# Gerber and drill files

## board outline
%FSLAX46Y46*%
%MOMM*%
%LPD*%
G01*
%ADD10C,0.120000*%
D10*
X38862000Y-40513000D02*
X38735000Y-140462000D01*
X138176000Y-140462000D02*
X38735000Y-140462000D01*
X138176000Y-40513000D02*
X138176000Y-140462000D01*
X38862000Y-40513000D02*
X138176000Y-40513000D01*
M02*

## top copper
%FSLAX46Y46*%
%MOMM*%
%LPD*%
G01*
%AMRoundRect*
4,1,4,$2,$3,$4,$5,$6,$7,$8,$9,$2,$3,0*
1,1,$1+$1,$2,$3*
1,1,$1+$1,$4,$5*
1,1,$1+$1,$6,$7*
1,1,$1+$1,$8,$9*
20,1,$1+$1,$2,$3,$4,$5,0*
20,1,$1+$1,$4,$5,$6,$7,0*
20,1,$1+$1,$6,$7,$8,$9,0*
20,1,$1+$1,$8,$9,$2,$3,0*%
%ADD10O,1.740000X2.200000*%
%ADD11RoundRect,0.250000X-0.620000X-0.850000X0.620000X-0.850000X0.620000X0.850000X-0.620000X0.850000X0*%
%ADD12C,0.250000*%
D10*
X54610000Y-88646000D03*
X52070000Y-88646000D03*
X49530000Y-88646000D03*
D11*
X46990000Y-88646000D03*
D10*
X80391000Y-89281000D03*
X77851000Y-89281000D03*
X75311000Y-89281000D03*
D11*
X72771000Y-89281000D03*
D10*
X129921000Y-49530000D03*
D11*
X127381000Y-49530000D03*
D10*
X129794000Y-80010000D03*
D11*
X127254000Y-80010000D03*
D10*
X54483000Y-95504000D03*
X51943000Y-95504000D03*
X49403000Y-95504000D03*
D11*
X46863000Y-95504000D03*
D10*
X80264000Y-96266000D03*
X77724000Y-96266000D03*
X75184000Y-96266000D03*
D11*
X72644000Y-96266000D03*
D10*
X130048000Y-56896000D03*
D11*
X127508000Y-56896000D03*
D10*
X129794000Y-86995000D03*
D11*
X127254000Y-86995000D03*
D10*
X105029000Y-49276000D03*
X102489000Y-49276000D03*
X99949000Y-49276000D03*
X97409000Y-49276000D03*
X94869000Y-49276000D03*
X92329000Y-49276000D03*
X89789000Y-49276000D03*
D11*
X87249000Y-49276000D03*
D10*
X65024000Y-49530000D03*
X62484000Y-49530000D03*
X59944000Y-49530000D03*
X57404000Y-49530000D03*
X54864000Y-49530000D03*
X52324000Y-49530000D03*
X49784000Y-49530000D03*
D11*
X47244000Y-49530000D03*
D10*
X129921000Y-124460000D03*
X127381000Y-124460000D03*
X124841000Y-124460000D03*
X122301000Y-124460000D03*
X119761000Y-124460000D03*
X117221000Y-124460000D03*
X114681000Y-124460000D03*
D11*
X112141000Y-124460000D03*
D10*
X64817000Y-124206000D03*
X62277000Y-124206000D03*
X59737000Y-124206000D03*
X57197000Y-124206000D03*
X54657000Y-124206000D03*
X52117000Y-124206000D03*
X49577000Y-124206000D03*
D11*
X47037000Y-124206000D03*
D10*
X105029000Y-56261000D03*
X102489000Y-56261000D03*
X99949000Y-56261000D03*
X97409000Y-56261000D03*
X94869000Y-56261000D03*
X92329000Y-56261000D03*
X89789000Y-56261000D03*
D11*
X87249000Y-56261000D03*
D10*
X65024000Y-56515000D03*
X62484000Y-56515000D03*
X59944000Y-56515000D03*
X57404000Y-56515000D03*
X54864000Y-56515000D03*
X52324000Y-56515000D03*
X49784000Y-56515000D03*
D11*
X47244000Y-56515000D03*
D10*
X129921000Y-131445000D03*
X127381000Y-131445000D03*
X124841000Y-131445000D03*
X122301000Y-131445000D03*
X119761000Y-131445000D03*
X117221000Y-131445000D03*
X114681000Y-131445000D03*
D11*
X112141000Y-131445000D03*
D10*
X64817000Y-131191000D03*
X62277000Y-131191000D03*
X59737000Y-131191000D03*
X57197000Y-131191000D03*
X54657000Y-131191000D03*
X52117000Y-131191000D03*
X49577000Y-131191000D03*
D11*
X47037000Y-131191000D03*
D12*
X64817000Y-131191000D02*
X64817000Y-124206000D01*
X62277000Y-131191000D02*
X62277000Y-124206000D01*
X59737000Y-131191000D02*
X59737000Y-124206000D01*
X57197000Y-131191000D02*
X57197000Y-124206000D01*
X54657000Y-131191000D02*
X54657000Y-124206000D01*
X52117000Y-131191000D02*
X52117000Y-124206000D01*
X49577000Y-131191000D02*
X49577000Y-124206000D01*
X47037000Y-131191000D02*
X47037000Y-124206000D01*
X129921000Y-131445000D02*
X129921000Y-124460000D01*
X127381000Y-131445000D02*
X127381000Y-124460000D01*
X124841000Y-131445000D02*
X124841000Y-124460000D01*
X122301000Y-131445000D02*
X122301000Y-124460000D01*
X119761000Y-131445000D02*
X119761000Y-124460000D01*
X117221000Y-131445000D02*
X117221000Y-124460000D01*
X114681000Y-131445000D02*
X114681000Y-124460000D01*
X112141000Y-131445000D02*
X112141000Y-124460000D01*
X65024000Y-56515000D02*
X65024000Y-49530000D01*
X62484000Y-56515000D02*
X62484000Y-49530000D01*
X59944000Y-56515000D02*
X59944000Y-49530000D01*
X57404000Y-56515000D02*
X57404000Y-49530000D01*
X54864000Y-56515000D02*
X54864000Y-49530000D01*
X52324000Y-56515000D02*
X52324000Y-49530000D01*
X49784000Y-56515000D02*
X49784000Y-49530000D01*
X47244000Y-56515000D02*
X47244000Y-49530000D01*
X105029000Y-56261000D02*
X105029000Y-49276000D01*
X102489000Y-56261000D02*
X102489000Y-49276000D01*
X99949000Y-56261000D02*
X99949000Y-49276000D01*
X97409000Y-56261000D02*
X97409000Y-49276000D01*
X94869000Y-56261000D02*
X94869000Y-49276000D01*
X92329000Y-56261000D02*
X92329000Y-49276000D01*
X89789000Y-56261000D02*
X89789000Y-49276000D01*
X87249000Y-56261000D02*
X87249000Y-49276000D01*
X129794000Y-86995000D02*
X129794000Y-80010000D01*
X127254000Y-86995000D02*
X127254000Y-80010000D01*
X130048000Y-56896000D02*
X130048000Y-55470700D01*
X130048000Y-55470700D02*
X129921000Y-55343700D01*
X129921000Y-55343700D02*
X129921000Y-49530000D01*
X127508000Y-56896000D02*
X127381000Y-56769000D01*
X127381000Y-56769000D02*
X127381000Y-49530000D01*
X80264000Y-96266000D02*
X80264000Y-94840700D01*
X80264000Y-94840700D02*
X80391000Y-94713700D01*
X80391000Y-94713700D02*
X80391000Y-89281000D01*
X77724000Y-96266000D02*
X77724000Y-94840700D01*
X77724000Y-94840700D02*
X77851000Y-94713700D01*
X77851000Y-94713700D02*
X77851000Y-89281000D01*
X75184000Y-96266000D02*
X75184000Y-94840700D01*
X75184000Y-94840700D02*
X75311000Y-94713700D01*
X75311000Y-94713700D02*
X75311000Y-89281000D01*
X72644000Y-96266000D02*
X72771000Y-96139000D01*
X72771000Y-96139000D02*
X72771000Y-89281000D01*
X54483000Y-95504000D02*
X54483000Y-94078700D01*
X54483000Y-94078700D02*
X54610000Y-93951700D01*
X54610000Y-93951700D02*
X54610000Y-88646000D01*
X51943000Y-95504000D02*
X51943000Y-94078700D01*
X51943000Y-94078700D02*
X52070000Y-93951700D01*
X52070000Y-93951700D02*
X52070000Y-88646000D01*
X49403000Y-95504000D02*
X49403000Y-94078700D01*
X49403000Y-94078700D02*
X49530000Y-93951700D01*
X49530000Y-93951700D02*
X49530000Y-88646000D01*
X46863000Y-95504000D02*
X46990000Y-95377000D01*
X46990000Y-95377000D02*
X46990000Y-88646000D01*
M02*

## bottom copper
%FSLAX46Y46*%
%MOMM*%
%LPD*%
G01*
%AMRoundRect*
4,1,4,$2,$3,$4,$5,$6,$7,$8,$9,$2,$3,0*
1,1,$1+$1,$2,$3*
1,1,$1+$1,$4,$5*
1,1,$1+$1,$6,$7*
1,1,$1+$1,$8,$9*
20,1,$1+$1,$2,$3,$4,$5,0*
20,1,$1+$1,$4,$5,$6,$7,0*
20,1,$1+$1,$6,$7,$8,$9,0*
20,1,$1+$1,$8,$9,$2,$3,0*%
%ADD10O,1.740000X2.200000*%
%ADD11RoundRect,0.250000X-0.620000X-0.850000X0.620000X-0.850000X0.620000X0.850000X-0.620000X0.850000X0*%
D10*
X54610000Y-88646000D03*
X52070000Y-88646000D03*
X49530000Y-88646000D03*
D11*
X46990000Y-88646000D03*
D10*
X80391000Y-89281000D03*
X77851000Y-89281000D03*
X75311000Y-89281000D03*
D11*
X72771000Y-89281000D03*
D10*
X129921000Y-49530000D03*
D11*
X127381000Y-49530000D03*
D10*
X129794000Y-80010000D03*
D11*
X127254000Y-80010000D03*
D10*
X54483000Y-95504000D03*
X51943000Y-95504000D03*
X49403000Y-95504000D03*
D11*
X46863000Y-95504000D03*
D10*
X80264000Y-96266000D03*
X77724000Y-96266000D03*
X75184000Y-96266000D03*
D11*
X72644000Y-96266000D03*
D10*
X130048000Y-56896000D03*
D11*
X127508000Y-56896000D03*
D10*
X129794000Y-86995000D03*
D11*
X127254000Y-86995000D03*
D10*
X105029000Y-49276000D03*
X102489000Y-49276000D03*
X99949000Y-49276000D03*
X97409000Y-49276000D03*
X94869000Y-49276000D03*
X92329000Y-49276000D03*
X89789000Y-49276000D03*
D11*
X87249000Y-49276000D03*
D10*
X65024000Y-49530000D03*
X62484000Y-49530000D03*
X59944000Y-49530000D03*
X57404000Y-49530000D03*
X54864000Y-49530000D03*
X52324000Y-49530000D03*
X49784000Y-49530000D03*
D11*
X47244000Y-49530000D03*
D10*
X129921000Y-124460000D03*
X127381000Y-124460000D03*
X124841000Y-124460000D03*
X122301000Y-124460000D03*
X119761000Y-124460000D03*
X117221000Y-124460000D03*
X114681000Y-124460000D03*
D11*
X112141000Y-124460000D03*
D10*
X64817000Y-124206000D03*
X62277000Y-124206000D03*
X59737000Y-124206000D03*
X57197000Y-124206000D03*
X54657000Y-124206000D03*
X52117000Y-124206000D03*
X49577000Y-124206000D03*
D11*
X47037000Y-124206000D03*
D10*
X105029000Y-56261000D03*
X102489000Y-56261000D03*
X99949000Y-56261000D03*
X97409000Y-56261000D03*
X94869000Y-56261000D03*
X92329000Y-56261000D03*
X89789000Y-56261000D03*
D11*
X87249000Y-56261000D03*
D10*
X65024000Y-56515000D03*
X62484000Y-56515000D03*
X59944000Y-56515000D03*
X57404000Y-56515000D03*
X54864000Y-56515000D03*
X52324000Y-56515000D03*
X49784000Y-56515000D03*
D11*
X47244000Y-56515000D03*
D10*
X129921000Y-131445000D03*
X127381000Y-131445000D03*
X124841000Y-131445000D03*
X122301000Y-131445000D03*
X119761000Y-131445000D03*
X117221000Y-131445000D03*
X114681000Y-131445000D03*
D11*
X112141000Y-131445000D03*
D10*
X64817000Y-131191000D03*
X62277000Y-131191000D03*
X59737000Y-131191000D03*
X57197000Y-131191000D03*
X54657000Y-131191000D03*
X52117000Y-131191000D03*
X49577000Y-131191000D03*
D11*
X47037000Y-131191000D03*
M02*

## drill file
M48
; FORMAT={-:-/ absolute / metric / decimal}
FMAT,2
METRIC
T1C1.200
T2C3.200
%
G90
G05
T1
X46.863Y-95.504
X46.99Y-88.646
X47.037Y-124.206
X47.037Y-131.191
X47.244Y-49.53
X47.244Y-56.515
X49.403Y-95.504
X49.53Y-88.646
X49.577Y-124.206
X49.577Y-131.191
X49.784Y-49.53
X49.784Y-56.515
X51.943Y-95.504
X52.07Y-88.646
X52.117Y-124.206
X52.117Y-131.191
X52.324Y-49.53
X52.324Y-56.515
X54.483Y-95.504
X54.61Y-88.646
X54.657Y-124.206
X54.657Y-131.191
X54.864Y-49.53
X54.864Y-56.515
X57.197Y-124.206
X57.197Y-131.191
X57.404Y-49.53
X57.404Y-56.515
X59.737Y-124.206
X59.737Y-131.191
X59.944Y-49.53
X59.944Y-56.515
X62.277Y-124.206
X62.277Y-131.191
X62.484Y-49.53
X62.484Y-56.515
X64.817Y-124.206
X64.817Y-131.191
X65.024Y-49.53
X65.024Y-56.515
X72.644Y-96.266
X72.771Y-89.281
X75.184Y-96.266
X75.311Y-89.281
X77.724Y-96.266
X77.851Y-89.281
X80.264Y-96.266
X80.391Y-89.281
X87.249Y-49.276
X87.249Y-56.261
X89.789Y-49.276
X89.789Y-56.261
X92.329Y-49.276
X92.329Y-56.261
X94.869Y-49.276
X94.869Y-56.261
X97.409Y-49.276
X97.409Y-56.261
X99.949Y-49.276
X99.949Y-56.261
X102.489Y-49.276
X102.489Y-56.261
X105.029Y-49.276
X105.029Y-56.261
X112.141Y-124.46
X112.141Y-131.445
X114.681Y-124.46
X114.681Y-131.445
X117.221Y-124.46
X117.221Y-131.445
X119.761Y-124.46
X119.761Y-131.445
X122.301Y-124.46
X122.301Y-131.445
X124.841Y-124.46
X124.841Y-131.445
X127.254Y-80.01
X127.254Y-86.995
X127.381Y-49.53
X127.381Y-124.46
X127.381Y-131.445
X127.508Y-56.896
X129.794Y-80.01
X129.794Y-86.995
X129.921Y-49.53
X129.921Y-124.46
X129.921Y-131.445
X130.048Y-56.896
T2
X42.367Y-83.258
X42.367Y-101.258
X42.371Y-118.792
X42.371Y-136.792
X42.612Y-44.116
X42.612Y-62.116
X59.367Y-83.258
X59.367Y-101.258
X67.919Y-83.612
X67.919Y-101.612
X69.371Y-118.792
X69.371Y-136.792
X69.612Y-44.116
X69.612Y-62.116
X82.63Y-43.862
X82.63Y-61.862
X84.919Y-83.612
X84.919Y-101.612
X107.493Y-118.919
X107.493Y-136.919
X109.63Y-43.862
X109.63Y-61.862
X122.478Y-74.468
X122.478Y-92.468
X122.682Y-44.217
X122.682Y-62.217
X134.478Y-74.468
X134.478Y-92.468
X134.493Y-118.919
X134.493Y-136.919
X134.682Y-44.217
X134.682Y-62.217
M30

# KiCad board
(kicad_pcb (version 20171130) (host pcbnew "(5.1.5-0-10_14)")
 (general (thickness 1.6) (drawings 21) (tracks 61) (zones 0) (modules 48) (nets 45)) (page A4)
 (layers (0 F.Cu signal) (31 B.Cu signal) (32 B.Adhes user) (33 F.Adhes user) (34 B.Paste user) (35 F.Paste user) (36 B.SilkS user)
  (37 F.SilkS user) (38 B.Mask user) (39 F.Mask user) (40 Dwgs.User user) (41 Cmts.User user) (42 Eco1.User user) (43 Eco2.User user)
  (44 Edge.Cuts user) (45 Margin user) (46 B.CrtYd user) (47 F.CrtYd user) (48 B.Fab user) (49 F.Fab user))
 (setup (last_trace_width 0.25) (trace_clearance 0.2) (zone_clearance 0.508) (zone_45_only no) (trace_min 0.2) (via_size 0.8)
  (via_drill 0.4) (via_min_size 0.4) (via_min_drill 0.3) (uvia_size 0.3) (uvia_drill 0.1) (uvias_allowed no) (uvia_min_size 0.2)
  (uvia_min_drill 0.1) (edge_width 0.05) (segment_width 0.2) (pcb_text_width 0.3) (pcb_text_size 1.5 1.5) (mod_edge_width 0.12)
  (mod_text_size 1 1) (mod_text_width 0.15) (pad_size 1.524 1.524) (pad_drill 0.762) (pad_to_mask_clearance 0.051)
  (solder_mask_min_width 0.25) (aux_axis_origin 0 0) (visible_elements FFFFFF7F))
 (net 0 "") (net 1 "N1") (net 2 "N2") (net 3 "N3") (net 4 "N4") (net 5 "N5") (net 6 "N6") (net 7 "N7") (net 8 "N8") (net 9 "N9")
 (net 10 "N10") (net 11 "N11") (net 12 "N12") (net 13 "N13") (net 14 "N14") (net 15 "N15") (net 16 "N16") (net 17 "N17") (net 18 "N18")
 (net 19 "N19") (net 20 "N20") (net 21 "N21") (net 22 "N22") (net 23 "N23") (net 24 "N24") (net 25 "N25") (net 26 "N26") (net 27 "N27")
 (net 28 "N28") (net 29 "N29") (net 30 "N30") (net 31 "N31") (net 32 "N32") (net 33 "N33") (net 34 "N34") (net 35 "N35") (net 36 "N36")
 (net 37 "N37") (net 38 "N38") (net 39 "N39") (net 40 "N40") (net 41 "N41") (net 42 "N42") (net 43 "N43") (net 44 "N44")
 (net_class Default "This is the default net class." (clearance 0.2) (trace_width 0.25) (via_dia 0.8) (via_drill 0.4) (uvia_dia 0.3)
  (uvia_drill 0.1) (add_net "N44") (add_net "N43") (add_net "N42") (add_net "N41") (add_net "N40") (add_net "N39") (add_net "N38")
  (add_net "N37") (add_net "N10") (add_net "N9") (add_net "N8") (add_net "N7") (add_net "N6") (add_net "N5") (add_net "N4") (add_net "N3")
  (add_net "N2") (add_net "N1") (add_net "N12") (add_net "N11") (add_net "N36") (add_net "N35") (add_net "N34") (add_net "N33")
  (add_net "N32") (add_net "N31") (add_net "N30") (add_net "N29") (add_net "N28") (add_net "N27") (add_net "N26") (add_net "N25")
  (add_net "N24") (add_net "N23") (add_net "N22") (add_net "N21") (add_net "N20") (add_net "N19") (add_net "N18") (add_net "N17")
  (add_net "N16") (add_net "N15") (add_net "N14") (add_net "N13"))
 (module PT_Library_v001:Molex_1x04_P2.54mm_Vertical (layer F.Cu) (at 46.99 88.646)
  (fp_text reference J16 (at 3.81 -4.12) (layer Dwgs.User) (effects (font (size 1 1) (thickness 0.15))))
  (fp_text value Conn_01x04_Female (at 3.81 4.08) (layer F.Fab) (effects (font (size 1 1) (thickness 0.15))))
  (pad 4 thru_hole oval (at 7.62 0) (size 1.74 2.2) (drill 1.2) (layers *.Cu *.Mask) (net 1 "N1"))
  (pad 3 thru_hole oval (at 5.08 0) (size 1.74 2.2) (drill 1.2) (layers *.Cu *.Mask) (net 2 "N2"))
  (pad 2 thru_hole oval (at 2.54 0) (size 1.74 2.2) (drill 1.2) (layers *.Cu *.Mask) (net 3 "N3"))
  (pad 1 thru_hole roundrect (at 0 0) (size 1.74 2.2) (drill 1.2) (layers *.Cu *.Mask) (roundrect_rratio 0.143678) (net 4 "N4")))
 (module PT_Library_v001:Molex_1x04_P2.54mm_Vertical (layer F.Cu) (at 72.771 89.281)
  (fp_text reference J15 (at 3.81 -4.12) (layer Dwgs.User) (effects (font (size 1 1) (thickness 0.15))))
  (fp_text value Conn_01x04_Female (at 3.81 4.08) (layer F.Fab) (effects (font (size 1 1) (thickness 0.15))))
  (pad 4 thru_hole oval (at 7.62 0) (size 1.74 2.2) (drill 1.2) (layers *.Cu *.Mask) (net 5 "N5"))
  (pad 3 thru_hole oval (at 5.08 0) (size 1.74 2.2) (drill 1.2) (layers *.Cu *.Mask) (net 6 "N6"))
  (pad 2 thru_hole oval (at 2.54 0) (size 1.74 2.2) (drill 1.2) (layers *.Cu *.Mask) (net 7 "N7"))
  (pad 1 thru_hole roundrect (at 0 0) (size 1.74 2.2) (drill 1.2) (layers *.Cu *.Mask) (roundrect_rratio 0.143678) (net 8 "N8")))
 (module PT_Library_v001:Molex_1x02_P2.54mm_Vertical (layer F.Cu) (at 127.381 49.53)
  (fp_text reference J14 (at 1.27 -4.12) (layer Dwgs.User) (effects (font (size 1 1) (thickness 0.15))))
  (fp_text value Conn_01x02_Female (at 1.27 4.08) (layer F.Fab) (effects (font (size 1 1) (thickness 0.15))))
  (pad 2 thru_hole oval (at 2.54 0) (size 1.74 2.2) (drill 1.2) (layers *.Cu *.Mask) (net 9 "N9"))
  (pad 1 thru_hole roundrect (at 0 0) (size 1.74 2.2) (drill 1.2) (layers *.Cu *.Mask) (roundrect_rratio 0.143678) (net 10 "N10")))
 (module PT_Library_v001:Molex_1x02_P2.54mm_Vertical (layer F.Cu) (at 127.254 80.01)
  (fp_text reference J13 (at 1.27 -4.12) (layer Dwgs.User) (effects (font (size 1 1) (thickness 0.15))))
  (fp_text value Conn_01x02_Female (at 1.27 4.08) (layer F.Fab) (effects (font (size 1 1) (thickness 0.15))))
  (pad 2 thru_hole oval (at 2.54 0) (size 1.74 2.2) (drill 1.2) (layers *.Cu *.Mask) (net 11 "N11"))
  (pad 1 thru_hole roundrect (at 0 0) (size 1.74 2.2) (drill 1.2) (layers *.Cu *.Mask) (roundrect_rratio 0.143678) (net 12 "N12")))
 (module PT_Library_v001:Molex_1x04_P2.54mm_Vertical (layer F.Cu) (at 46.863 95.504)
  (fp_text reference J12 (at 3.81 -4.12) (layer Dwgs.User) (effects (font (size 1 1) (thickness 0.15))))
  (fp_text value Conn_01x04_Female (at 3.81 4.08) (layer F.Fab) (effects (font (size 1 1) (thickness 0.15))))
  (pad 4 thru_hole oval (at 7.62 0) (size 1.74 2.2) (drill 1.2) (layers *.Cu *.Mask) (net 1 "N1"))
  (pad 3 thru_hole oval (at 5.08 0) (size 1.74 2.2) (drill 1.2) (layers *.Cu *.Mask) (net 2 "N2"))
  (pad 2 thru_hole oval (at 2.54 0) (size 1.74 2.2) (drill 1.2) (layers *.Cu *.Mask) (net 3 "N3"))
  (pad 1 thru_hole roundrect (at 0 0) (size 1.74 2.2) (drill 1.2) (layers *.Cu *.Mask) (roundrect_rratio 0.143678) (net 4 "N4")))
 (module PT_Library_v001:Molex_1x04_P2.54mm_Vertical (layer F.Cu) (at 72.644 96.266)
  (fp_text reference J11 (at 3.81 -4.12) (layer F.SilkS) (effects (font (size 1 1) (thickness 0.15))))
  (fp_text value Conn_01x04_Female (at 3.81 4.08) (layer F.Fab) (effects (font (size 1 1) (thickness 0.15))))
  (pad 4 thru_hole oval (at 7.62 0) (size 1.74 2.2) (drill 1.2) (layers *.Cu *.Mask) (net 5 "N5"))
  (pad 3 thru_hole oval (at 5.08 0) (size 1.74 2.2) (drill 1.2) (layers *.Cu *.Mask) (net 6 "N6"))
  (pad 2 thru_hole oval (at 2.54 0) (size 1.74 2.2) (drill 1.2) (layers *.Cu *.Mask) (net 7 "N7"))
  (pad 1 thru_hole roundrect (at 0 0) (size 1.74 2.2) (drill 1.2) (layers *.Cu *.Mask) (roundrect_rratio 0.143678) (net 8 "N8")))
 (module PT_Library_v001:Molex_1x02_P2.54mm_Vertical (layer F.Cu) (at 127.508 56.896)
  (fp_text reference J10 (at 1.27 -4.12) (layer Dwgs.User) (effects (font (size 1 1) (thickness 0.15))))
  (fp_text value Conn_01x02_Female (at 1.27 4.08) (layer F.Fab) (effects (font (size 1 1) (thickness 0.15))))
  (pad 2 thru_hole oval (at 2.54 0) (size 1.74 2.2) (drill 1.2) (layers *.Cu *.Mask) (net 9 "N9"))
  (pad 1 thru_hole roundrect (at 0 0) (size 1.74 2.2) (drill 1.2) (layers *.Cu *.Mask) (roundrect_rratio 0.143678) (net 10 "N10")))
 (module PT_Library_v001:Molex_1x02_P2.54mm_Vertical (layer F.Cu) (at 127.254 86.995)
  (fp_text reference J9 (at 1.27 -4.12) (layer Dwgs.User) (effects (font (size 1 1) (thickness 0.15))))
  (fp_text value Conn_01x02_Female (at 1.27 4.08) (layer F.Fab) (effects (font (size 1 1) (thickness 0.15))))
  (pad 2 thru_hole oval (at 2.54 0) (size 1.74 2.2) (drill 1.2) (layers *.Cu *.Mask) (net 11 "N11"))
  (pad 1 thru_hole roundrect (at 0 0) (size 1.74 2.2) (drill 1.2) (layers *.Cu *.Mask) (roundrect_rratio 0.143678) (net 12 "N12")))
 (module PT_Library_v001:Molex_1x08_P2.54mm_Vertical (layer F.Cu) (at 87.249 49.276)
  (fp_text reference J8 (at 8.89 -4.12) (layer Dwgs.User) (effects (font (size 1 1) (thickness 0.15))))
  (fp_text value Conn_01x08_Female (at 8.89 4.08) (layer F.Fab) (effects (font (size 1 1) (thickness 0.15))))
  (pad 8 thru_hole oval (at 17.78 0) (size 1.74 2.2) (drill 1.2) (layers *.Cu *.Mask) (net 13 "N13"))
  (pad 7 thru_hole oval (at 15.24 0) (size 1.74 2.2) (drill 1.2) (layers *.Cu *.Mask) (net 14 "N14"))
  (pad 6 thru_hole oval (at 12.7 0) (size 1.74 2.2) (drill 1.2) (layers *.Cu *.Mask) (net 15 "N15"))
  (pad 5 thru_hole oval (at 10.16 0) (size 1.74 2.2) (drill 1.2) (layers *.Cu *.Mask) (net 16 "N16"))
  (pad 4 thru_hole oval (at 7.62 0) (size 1.74 2.2) (drill 1.2) (layers *.Cu *.Mask) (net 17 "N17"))
  (pad 3 thru_hole oval (at 5.08 0) (size 1.74 2.2) (drill 1.2) (layers *.Cu *.Mask) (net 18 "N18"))
  (pad 2 thru_hole oval (at 2.54 0) (size 1.74 2.2) (drill 1.2) (layers *.Cu *.Mask) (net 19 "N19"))
  (pad 1 thru_hole roundrect (at 0 0) (size 1.74 2.2) (drill 1.2) (layers *.Cu *.Mask) (roundrect_rratio 0.143678) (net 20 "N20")))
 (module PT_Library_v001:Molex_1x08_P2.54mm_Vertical (layer F.Cu) (at 47.244 49.53)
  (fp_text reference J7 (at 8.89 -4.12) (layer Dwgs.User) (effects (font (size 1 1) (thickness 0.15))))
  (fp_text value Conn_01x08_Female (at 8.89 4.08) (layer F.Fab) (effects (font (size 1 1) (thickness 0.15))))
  (pad 8 thru_hole oval (at 17.78 0) (size 1.74 2.2) (drill 1.2) (layers *.Cu *.Mask) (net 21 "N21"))
  (pad 7 thru_hole oval (at 15.24 0) (size 1.74 2.2) (drill 1.2) (layers *.Cu *.Mask) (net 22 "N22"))
  (pad 6 thru_hole oval (at 12.7 0) (size 1.74 2.2) (drill 1.2) (layers *.Cu *.Mask) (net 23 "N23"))
  (pad 5 thru_hole oval (at 10.16 0) (size 1.74 2.2) (drill 1.2) (layers *.Cu *.Mask) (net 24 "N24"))
  (pad 4 thru_hole oval (at 7.62 0) (size 1.74 2.2) (drill 1.2) (layers *.Cu *.Mask) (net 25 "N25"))
  (pad 3 thru_hole oval (at 5.08 0) (size 1.74 2.2) (drill 1.2) (layers *.Cu *.Mask) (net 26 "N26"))
  (pad 2 thru_hole oval (at 2.54 0) (size 1.74 2.2) (drill 1.2) (layers *.Cu *.Mask) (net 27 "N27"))
  (pad 1 thru_hole roundrect (at 0 0) (size 1.74 2.2) (drill 1.2) (layers *.Cu *.Mask) (roundrect_rratio 0.143678) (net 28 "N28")))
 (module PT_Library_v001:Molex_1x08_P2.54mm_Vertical (layer F.Cu) (at 112.141 124.46)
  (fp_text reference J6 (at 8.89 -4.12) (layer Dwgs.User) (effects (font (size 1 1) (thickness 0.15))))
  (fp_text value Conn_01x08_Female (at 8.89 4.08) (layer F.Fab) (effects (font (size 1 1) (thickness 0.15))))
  (pad 8 thru_hole oval (at 17.78 0) (size 1.74 2.2) (drill 1.2) (layers *.Cu *.Mask) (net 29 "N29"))
  (pad 7 thru_hole oval (at 15.24 0) (size 1.74 2.2) (drill 1.2) (layers *.Cu *.Mask) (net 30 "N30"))
  (pad 6 thru_hole oval (at 12.7 0) (size 1.74 2.2) (drill 1.2) (layers *.Cu *.Mask) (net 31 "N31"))
  (pad 5 thru_hole oval (at 10.16 0) (size 1.74 2.2) (drill 1.2) (layers *.Cu *.Mask) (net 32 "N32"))
  (pad 4 thru_hole oval (at 7.62 0) (size 1.74 2.2) (drill 1.2) (layers *.Cu *.Mask) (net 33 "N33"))
  (pad 3 thru_hole oval (at 5.08 0) (size 1.74 2.2) (drill 1.2) (layers *.Cu *.Mask) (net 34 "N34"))
  (pad 2 thru_hole oval (at 2.54 0) (size 1.74 2.2) (drill 1.2) (layers *.Cu *.Mask) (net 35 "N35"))
  (pad 1 thru_hole roundrect (at 0 0) (size 1.74 2.2) (drill 1.2) (layers *.Cu *.Mask) (roundrect_rratio 0.143678) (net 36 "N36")))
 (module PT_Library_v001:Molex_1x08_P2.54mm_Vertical (layer F.Cu) (at 47.037 124.206)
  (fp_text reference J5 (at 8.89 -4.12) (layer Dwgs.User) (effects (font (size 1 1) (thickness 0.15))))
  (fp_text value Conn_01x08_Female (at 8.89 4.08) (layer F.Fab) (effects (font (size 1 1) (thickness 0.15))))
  (pad 8 thru_hole oval (at 17.78 0) (size 1.74 2.2) (drill 1.2) (layers *.Cu *.Mask) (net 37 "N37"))
  (pad 7 thru_hole oval (at 15.24 0) (size 1.74 2.2) (drill 1.2) (layers *.Cu *.Mask) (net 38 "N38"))
  (pad 6 thru_hole oval (at 12.7 0) (size 1.74 2.2) (drill 1.2) (layers *.Cu *.Mask) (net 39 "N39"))
  (pad 5 thru_hole oval (at 10.16 0) (size 1.74 2.2) (drill 1.2) (layers *.Cu *.Mask) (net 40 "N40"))
  (pad 4 thru_hole oval (at 7.62 0) (size 1.74 2.2) (drill 1.2) (layers *.Cu *.Mask) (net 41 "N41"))
  (pad 3 thru_hole oval (at 5.08 0) (size 1.74 2.2) (drill 1.2) (layers *.Cu *.Mask) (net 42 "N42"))
  (pad 2 thru_hole oval (at 2.54 0) (size 1.74 2.2) (drill 1.2) (layers *.Cu *.Mask) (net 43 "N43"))
  (pad 1 thru_hole roundrect (at 0 0) (size 1.74 2.2) (drill 1.2) (layers *.Cu *.Mask) (roundrect_rratio 0.143678) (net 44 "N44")))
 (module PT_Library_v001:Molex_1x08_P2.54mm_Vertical (layer F.Cu) (at 87.249 56.261)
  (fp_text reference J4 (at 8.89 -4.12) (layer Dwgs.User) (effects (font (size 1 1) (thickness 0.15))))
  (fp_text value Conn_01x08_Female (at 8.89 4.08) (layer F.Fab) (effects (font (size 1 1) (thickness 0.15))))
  (pad 8 thru_hole oval (at 17.78 0) (size 1.74 2.2) (drill 1.2) (layers *.Cu *.Mask) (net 13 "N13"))
  (pad 7 thru_hole oval (at 15.24 0) (size 1.74 2.2) (drill 1.2) (layers *.Cu *.Mask) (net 14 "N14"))
  (pad 6 thru_hole oval (at 12.7 0) (size 1.74 2.2) (drill 1.2) (layers *.Cu *.Mask) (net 15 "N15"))
  (pad 5 thru_hole oval (at 10.16 0) (size 1.74 2.2) (drill 1.2) (layers *.Cu *.Mask) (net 16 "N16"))
  (pad 4 thru_hole oval (at 7.62 0) (size 1.74 2.2) (drill 1.2) (layers *.Cu *.Mask) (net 17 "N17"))
  (pad 3 thru_hole oval (at 5.08 0) (size 1.74 2.2) (drill 1.2) (layers *.Cu *.Mask) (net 18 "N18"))
  (pad 2 thru_hole oval (at 2.54 0) (size 1.74 2.2) (drill 1.2) (layers *.Cu *.Mask) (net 19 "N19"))
  (pad 1 thru_hole roundrect (at 0 0) (size 1.74 2.2) (drill 1.2) (layers *.Cu *.Mask) (roundrect_rratio 0.143678) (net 20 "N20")))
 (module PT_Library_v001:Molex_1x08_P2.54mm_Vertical (layer F.Cu) (at 47.244 56.515)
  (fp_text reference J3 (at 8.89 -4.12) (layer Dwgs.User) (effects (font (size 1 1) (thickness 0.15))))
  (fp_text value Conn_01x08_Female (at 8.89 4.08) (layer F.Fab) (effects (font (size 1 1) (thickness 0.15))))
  (pad 8 thru_hole oval (at 17.78 0) (size 1.74 2.2) (drill 1.2) (layers *.Cu *.Mask) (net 21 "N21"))
  (pad 7 thru_hole oval (at 15.24 0) (size 1.74 2.2) (drill 1.2) (layers *.Cu *.Mask) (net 22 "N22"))
  (pad 6 thru_hole oval (at 12.7 0) (size 1.74 2.2) (drill 1.2) (layers *.Cu *.Mask) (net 23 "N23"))
  (pad 5 thru_hole oval (at 10.16 0) (size 1.74 2.2) (drill 1.2) (layers *.Cu *.Mask) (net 24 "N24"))
  (pad 4 thru_hole oval (at 7.62 0) (size 1.74 2.2) (drill 1.2) (layers *.Cu *.Mask) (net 25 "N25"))
  (pad 3 thru_hole oval (at 5.08 0) (size 1.74 2.2) (drill 1.2) (layers *.Cu *.Mask) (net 26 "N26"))
  (pad 2 thru_hole oval (at 2.54 0) (size 1.74 2.2) (drill 1.2) (layers *.Cu *.Mask) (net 27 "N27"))
  (pad 1 thru_hole roundrect (at 0 0) (size 1.74 2.2) (drill 1.2) (layers *.Cu *.Mask) (roundrect_rratio 0.143678) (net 28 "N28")))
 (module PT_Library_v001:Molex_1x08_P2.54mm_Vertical (layer F.Cu) (at 112.141 131.445)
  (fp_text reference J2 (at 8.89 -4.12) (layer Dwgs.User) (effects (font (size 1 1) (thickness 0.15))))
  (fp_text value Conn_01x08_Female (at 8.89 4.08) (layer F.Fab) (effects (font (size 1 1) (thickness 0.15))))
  (pad 8 thru_hole oval (at 17.78 0) (size 1.74 2.2) (drill 1.2) (layers *.Cu *.Mask) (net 29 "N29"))
  (pad 7 thru_hole oval (at 15.24 0) (size 1.74 2.2) (drill 1.2) (layers *.Cu *.Mask) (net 30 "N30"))
  (pad 6 thru_hole oval (at 12.7 0) (size 1.74 2.2) (drill 1.2) (layers *.Cu *.Mask) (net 31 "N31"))
  (pad 5 thru_hole oval (at 10.16 0) (size 1.74 2.2) (drill 1.2) (layers *.Cu *.Mask) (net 32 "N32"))
  (pad 4 thru_hole oval (at 7.62 0) (size 1.74 2.2) (drill 1.2) (layers *.Cu *.Mask) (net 33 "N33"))
  (pad 3 thru_hole oval (at 5.08 0) (size 1.74 2.2) (drill 1.2) (layers *.Cu *.Mask) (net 34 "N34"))
  (pad 2 thru_hole oval (at 2.54 0) (size 1.74 2.2) (drill 1.2) (layers *.Cu *.Mask) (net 35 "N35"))
  (pad 1 thru_hole roundrect (at 0 0) (size 1.74 2.2) (drill 1.2) (layers *.Cu *.Mask) (roundrect_rratio 0.143678) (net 36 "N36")))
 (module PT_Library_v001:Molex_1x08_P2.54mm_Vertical (layer F.Cu) (at 47.037 131.191)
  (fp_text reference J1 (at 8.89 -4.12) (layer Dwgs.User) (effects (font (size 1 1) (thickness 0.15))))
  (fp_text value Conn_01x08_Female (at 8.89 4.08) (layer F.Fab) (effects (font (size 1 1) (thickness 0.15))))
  (pad 8 thru_hole oval (at 17.78 0) (size 1.74 2.2) (drill 1.2) (layers *.Cu *.Mask) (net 37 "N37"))
  (pad 7 thru_hole oval (at 15.24 0) (size 1.74 2.2) (drill 1.2) (layers *.Cu *.Mask) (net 38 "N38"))
  (pad 6 thru_hole oval (at 12.7 0) (size 1.74 2.2) (drill 1.2) (layers *.Cu *.Mask) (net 39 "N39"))
  (pad 5 thru_hole oval (at 10.16 0) (size 1.74 2.2) (drill 1.2) (layers *.Cu *.Mask) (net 40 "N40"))
  (pad 4 thru_hole oval (at 7.62 0) (size 1.74 2.2) (drill 1.2) (layers *.Cu *.Mask) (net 41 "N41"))
  (pad 3 thru_hole oval (at 5.08 0) (size 1.74 2.2) (drill 1.2) (layers *.Cu *.Mask) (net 42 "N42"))
  (pad 2 thru_hole oval (at 2.54 0) (size 1.74 2.2) (drill 1.2) (layers *.Cu *.Mask) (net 43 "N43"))
  (pad 1 thru_hole roundrect (at 0 0) (size 1.74 2.2) (drill 1.2) (layers *.Cu *.Mask) (roundrect_rratio 0.143678) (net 44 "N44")))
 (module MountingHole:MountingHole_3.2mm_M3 (layer F.Cu) (at 42.367 83.258)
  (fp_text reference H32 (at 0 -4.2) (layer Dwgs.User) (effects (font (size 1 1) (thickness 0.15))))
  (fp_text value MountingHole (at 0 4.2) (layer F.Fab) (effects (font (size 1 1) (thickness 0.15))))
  (pad 1 np_thru_hole circle (at 0 0) (size 3.2 3.2) (drill 3.2) (layers *.Cu *.Mask)))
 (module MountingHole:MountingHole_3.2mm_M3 (layer F.Cu) (at 42.371 118.792)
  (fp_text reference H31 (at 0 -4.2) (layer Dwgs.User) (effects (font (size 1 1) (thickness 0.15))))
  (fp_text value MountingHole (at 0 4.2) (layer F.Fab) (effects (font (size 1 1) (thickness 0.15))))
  (pad 1 np_thru_hole circle (at 0 0) (size 3.2 3.2) (drill 3.2) (layers *.Cu *.Mask)))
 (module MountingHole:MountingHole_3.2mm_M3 (layer F.Cu) (at 42.367 101.258)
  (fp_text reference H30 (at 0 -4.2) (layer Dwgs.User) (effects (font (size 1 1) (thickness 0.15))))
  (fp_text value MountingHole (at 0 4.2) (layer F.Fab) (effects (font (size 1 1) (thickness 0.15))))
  (pad 1 np_thru_hole circle (at 0 0) (size 3.2 3.2) (drill 3.2) (layers *.Cu *.Mask)))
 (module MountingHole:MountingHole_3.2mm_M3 (layer F.Cu) (at 122.682 44.217)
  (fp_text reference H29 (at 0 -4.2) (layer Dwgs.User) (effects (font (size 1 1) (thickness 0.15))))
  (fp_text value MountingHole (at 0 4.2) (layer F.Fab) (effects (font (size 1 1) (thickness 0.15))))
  (pad 1 np_thru_hole circle (at 0 0) (size 3.2 3.2) (drill 3.2) (layers *.Cu *.Mask)))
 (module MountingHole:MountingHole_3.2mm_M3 (layer F.Cu) (at 122.478 74.468)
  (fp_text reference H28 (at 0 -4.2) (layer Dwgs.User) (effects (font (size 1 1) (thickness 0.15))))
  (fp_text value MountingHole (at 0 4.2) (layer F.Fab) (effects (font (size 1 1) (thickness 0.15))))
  (pad 1 np_thru_hole circle (at 0 0) (size 3.2 3.2) (drill 3.2) (layers *.Cu *.Mask)))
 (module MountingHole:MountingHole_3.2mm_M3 (layer F.Cu) (at 69.371 118.792)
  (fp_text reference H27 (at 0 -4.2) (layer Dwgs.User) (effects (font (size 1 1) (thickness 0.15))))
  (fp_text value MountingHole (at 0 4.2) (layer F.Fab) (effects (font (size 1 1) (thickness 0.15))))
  (pad 1 np_thru_hole circle (at 0 0) (size 3.2 3.2) (drill 3.2) (layers *.Cu *.Mask)))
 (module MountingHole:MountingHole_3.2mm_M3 (layer F.Cu) (at 67.919 83.612)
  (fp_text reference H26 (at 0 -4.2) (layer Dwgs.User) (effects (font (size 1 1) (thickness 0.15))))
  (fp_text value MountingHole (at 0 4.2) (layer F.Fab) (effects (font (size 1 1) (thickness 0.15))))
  (pad 1 np_thru_hole circle (at 0 0) (size 3.2 3.2) (drill 3.2) (layers *.Cu *.Mask)))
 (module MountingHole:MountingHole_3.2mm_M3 (layer F.Cu) (at 122.478 92.468)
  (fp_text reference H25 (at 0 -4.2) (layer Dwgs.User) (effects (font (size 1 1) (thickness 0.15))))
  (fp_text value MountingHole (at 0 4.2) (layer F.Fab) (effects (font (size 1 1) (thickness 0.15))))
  (pad 1 np_thru_hole circle (at 0 0) (size 3.2 3.2) (drill 3.2) (layers *.Cu *.Mask)))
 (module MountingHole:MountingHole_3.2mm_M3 (layer F.Cu) (at 59.367 101.258)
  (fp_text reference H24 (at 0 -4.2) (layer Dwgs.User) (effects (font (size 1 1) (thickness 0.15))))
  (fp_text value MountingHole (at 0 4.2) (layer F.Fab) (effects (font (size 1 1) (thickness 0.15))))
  (pad 1 np_thru_hole circle (at 0 0) (size 3.2 3.2) (drill 3.2) (layers *.Cu *.Mask)))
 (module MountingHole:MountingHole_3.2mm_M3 (layer F.Cu) (at 107.493 118.919)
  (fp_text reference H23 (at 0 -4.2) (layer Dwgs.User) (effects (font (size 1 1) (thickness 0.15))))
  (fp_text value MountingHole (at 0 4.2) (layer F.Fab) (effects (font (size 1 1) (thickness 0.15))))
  (pad 1 np_thru_hole circle (at 0 0) (size 3.2 3.2) (drill 3.2) (layers *.Cu *.Mask)))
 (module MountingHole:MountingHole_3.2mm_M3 (layer F.Cu) (at 42.612 44.116)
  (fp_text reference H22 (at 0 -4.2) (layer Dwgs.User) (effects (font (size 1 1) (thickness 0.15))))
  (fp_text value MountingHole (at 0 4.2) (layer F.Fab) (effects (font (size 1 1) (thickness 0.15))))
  (pad 1 np_thru_hole circle (at 0 0) (size 3.2 3.2) (drill 3.2) (layers *.Cu *.Mask)))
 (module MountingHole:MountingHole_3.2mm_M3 (layer F.Cu) (at 82.63 43.862)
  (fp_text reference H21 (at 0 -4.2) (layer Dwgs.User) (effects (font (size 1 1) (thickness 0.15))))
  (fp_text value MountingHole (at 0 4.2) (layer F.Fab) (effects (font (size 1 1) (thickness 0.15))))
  (pad 1 np_thru_hole circle (at 0 0) (size 3.2 3.2) (drill 3.2) (layers *.Cu *.Mask)))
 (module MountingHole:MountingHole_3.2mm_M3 (layer F.Cu) (at 107.493 136.919)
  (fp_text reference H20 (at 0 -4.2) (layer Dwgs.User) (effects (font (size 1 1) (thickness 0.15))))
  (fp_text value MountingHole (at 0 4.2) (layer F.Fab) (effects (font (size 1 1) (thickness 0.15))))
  (pad 1 np_thru_hole circle (at 0 0) (size 3.2 3.2) (drill 3.2) (layers *.Cu *.Mask)))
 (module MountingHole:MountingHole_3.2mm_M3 (layer F.Cu) (at 82.63 61.862)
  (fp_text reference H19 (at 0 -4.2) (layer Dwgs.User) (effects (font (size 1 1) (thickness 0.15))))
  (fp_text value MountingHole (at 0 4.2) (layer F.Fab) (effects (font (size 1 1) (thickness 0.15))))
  (pad 1 np_thru_hole circle (at 0 0) (size 3.2 3.2) (drill 3.2) (layers *.Cu *.Mask)))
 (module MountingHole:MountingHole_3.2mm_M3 (layer F.Cu) (at 109.63 43.862)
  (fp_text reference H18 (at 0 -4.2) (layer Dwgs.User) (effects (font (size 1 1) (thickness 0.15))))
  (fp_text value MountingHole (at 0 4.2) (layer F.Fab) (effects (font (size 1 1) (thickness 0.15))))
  (pad 1 np_thru_hole circle (at 0 0) (size 3.2 3.2) (drill 3.2) (layers *.Cu *.Mask)))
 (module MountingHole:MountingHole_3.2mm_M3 (layer F.Cu) (at 134.493 118.919)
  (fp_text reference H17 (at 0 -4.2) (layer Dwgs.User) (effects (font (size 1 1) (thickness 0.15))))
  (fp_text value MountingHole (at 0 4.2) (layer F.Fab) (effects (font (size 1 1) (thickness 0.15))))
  (pad 1 np_thru_hole circle (at 0 0) (size 3.2 3.2) (drill 3.2) (layers *.Cu *.Mask)))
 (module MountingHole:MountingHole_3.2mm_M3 (layer F.Cu) (at 42.612 62.116)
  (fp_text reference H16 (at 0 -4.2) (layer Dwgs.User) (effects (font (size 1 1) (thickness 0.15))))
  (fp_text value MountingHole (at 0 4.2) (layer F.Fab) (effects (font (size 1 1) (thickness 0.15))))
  (pad 1 np_thru_hole circle (at 0 0) (size 3.2 3.2) (drill 3.2) (layers *.Cu *.Mask)))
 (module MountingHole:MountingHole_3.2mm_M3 (layer F.Cu) (at 109.63 61.862)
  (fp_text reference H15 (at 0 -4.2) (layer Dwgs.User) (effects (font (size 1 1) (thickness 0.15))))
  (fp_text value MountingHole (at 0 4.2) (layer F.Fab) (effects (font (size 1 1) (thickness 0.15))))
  (pad 1 np_thru_hole circle (at 0 0) (size 3.2 3.2) (drill 3.2) (layers *.Cu *.Mask)))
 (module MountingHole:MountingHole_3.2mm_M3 (layer F.Cu) (at 69.612 44.116)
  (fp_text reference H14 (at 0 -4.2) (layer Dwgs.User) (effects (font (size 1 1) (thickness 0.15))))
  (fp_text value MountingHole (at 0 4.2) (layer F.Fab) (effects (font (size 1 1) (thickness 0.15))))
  (pad 1 np_thru_hole circle (at 0 0) (size 3.2 3.2) (drill 3.2) (layers *.Cu *.Mask)))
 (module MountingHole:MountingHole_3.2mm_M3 (layer F.Cu) (at 69.612 62.116)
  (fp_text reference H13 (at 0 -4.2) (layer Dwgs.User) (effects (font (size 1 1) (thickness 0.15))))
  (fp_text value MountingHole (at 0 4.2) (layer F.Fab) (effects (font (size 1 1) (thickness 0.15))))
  (pad 1 np_thru_hole circle (at 0 0) (size 3.2 3.2) (drill 3.2) (layers *.Cu *.Mask)))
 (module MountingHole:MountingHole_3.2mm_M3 (layer F.Cu) (at 42.371 136.792)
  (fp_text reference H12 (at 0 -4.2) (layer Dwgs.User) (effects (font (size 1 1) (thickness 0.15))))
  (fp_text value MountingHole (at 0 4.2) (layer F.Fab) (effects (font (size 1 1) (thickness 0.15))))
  (pad 1 np_thru_hole circle (at 0 0) (size 3.2 3.2) (drill 3.2) (layers *.Cu *.Mask)))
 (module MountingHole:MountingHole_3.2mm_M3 (layer F.Cu) (at 67.919 101.612)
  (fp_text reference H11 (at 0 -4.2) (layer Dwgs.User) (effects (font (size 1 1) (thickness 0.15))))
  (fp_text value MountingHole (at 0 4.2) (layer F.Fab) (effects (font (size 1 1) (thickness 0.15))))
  (pad 1 np_thru_hole circle (at 0 0) (size 3.2 3.2) (drill 3.2) (layers *.Cu *.Mask)))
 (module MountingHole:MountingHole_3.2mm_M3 (layer F.Cu) (at 122.682 62.217)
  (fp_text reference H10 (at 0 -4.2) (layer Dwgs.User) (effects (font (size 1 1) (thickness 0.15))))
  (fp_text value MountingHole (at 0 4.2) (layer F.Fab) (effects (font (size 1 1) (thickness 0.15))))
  (pad 1 np_thru_hole circle (at 0 0) (size 3.2 3.2) (drill 3.2) (layers *.Cu *.Mask)))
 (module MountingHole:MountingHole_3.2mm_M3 (layer F.Cu) (at 134.478 74.468)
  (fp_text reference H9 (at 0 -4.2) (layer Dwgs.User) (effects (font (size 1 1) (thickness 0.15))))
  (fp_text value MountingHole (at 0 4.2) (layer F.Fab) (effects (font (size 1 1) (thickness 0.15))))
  (pad 1 np_thru_hole circle (at 0 0) (size 3.2 3.2) (drill 3.2) (layers *.Cu *.Mask)))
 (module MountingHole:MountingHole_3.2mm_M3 (layer F.Cu) (at 84.919 83.612)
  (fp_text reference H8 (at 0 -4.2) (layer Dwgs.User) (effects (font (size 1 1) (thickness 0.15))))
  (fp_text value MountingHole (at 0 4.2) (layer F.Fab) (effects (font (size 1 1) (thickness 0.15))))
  (pad 1 np_thru_hole circle (at 0 0) (size 3.2 3.2) (drill 3.2) (layers *.Cu *.Mask)))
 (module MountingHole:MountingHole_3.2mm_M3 (layer F.Cu) (at 59.367 83.258)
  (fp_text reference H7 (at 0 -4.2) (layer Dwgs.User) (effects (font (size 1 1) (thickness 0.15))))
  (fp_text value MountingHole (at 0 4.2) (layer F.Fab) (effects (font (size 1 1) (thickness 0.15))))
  (pad 1 np_thru_hole circle (at 0 0) (size 3.2 3.2) (drill 3.2) (layers *.Cu *.Mask)))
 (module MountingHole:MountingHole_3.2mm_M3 (layer F.Cu) (at 69.371 136.792)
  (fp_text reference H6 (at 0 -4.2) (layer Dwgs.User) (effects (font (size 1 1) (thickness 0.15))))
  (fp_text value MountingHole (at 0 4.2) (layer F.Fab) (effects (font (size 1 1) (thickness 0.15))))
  (pad 1 np_thru_hole circle (at 0 0) (size 3.2 3.2) (drill 3.2) (layers *.Cu *.Mask)))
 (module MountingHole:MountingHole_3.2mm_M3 (layer F.Cu) (at 134.682 44.217)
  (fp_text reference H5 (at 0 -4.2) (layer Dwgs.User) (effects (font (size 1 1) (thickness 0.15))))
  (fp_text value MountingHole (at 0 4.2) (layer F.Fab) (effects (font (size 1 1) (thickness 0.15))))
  (pad 1 np_thru_hole circle (at 0 0) (size 3.2 3.2) (drill 3.2) (layers *.Cu *.Mask)))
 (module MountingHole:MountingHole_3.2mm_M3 (layer F.Cu) (at 84.919 101.612)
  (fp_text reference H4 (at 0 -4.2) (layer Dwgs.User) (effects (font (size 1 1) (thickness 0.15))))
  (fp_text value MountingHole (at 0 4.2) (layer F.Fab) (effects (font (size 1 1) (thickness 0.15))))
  (pad 1 np_thru_hole circle (at 0 0) (size 3.2 3.2) (drill 3.2) (layers *.Cu *.Mask)))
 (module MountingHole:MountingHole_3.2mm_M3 (layer F.Cu) (at 134.478 92.468)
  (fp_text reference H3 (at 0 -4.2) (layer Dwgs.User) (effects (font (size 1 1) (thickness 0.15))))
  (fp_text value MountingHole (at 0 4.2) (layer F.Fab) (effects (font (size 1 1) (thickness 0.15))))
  (pad 1 np_thru_hole circle (at 0 0) (size 3.2 3.2) (drill 3.2) (layers *.Cu *.Mask)))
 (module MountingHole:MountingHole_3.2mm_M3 (layer F.Cu) (at 134.682 62.217)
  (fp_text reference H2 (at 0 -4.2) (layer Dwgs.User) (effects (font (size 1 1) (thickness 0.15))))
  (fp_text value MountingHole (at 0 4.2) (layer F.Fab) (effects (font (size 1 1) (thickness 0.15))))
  (pad 1 np_thru_hole circle (at 0 0) (size 3.2 3.2) (drill 3.2) (layers *.Cu *.Mask)))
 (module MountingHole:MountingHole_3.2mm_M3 (layer F.Cu) (at 134.493 136.919)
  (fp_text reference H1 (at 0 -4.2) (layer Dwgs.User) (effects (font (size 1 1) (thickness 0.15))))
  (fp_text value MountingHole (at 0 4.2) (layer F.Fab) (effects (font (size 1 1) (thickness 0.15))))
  (pad 1 np_thru_hole circle (at 0 0) (size 3.2 3.2) (drill 3.2) (layers *.Cu *.Mask)))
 (gr_line (start 38.862 40.513) (end 38.735 140.462) (layer Edge.Cuts) (width 0.12))
 (gr_line (start 138.176 140.462) (end 38.735 140.462) (layer Edge.Cuts) (width 0.12))
 (gr_line (start 138.176 40.513) (end 138.176 140.462) (layer Edge.Cuts) (width 0.12))
 (gr_line (start 38.862 40.513) (end 138.176 40.513) (layer Edge.Cuts) (width 0.12))
 (segment (start 64.817 131.191) (end 64.817 124.206) (width 0.25) (layer F.Cu) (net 37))
 (segment (start 62.277 131.191) (end 62.277 124.206) (width 0.25) (layer F.Cu) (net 38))
 (segment (start 59.737 131.191) (end 59.737 124.206) (width 0.25) (layer F.Cu) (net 39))
 (segment (start 57.197 131.191) (end 57.197 124.206) (width 0.25) (layer F.Cu) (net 40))
 (segment (start 54.657 131.191) (end 54.657 124.206) (width 0.25) (layer F.Cu) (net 41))
 (segment (start 52.117 131.191) (end 52.117 124.206) (width 0.25) (layer F.Cu) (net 42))
 (segment (start 49.577 131.191) (end 49.577 124.206) (width 0.25) (layer F.Cu) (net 43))
 (segment (start 47.037 131.191) (end 47.037 124.206) (width 0.25) (layer F.Cu) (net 44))
 (segment (start 129.921 131.445) (end 129.921 124.46) (width 0.25) (layer F.Cu) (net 29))
 (segment (start 127.381 131.445) (end 127.381 124.46) (width 0.25) (layer F.Cu) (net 30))
 (segment (start 124.841 131.445) (end 124.841 124.46) (width 0.25) (layer F.Cu) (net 31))
 (segment (start 122.301 131.445) (end 122.301 124.46) (width 0.25) (layer F.Cu) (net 32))
 (segment (start 119.761 131.445) (end 119.761 124.46) (width 0.25) (layer F.Cu) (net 33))
 (segment (start 117.221 131.445) (end 117.221 124.46) (width 0.25) (layer F.Cu) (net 34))
 (segment (start 114.681 131.445) (end 114.681 124.46) (width 0.25) (layer F.Cu) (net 35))
 (segment (start 112.141 131.445) (end 112.141 124.46) (width 0.25) (layer F.Cu) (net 36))
 (segment (start 65.024 56.515) (end 65.024 49.53) (width 0.25) (layer F.Cu) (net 21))
 (segment (start 62.484 56.515) (end 62.484 49.53) (width 0.25) (layer F.Cu) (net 22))
 (segment (start 59.944 56.515) (end 59.944 49.53) (width 0.25) (layer F.Cu) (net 23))
 (segment (start 57.404 56.515) (end 57.404 49.53) (width 0.25) (layer F.Cu) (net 24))
 (segment (start 54.864 56.515) (end 54.864 49.53) (width 0.25) (layer F.Cu) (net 25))
 (segment (start 52.324 56.515) (end 52.324 49.53) (width 0.25) (layer F.Cu) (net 26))
 (segment (start 49.784 56.515) (end 49.784 49.53) (width 0.25) (layer F.Cu) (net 27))
 (segment (start 47.244 56.515) (end 47.244 49.53) (width 0.25) (layer F.Cu) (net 28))
 (segment (start 105.029 56.261) (end 105.029 49.276) (width 0.25) (layer F.Cu) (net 13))
 (segment (start 102.489 56.261) (end 102.489 49.276) (width 0.25) (layer F.Cu) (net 14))
 (segment (start 99.949 56.261) (end 99.949 49.276) (width 0.25) (layer F.Cu) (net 15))
 (segment (start 97.409 56.261) (end 97.409 49.276) (width 0.25) (layer F.Cu) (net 16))
 (segment (start 94.869 56.261) (end 94.869 49.276) (width 0.25) (layer F.Cu) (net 17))
 (segment (start 92.329 56.261) (end 92.329 49.276) (width 0.25) (layer F.Cu) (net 18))
 (segment (start 89.789 56.261) (end 89.789 49.276) (width 0.25) (layer F.Cu) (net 19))
 (segment (start 87.249 56.261) (end 87.249 49.276) (width 0.25) (layer F.Cu) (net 20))
 (segment (start 129.794 86.995) (end 129.794 80.01) (width 0.25) (layer F.Cu) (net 11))
 (segment (start 127.254 86.995) (end 127.254 80.01) (width 0.25) (layer F.Cu) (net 12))
 (segment (start 130.048 56.896) (end 130.048 55.4707) (width 0.25) (layer F.Cu) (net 9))
 (segment (start 130.048 55.4707) (end 129.921 55.3437) (width 0.25) (layer F.Cu) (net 9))
 (segment (start 129.921 55.3437) (end 129.921 49.53) (width 0.25) (layer F.Cu) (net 9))
 (segment (start 127.508 56.896) (end 127.381 56.769) (width 0.25) (layer F.Cu) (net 10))
 (segment (start 127.381 56.769) (end 127.381 49.53) (width 0.25) (layer F.Cu) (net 10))
 (segment (start 80.264 96.266) (end 80.264 94.8407) (width 0.25) (layer F.Cu) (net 5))
 (segment (start 80.264 94.8407) (end 80.391 94.7137) (width 0.25) (layer F.Cu) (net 5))
 (segment (start 80.391 94.7137) (end 80.391 89.281) (width 0.25) (layer F.Cu) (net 5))
 (segment (start 77.724 96.266) (end 77.724 94.8407) (width 0.25) (layer F.Cu) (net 6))
 (segment (start 77.724 94.8407) (end 77.851 94.7137) (width 0.25) (layer F.Cu) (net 6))
 (segment (start 77.851 94.7137) (end 77.851 89.281) (width 0.25) (layer F.Cu) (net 6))
 (segment (start 75.184 96.266) (end 75.184 94.8407) (width 0.25) (layer F.Cu) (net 7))
 (segment (start 75.184 94.8407) (end 75.311 94.7137) (width 0.25) (layer F.Cu) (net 7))
 (segment (start 75.311 94.7137) (end 75.311 89.281) (width 0.25) (layer F.Cu) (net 7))
 (segment (start 72.644 96.266) (end 72.771 96.139) (width 0.25) (layer F.Cu) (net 8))
 (segment (start 72.771 96.139) (end 72.771 89.281) (width 0.25) (layer F.Cu) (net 8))
 (segment (start 54.483 95.504) (end 54.483 94.0787) (width 0.25) (layer F.Cu) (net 1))
 (segment (start 54.483 94.0787) (end 54.61 93.9517) (width 0.25) (layer F.Cu) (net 1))
 (segment (start 54.61 93.9517) (end 54.61 88.646) (width 0.25) (layer F.Cu) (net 1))
 (segment (start 51.943 95.504) (end 51.943 94.0787) (width 0.25) (layer F.Cu) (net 2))
 (segment (start 51.943 94.0787) (end 52.07 93.9517) (width 0.25) (layer F.Cu) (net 2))
 (segment (start 52.07 93.9517) (end 52.07 88.646) (width 0.25) (layer F.Cu) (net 2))
 (segment (start 49.403 95.504) (end 49.403 94.0787) (width 0.25) (layer F.Cu) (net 3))
 (segment (start 49.403 94.0787) (end 49.53 93.9517) (width 0.25) (layer F.Cu) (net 3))
 (segment (start 49.53 93.9517) (end 49.53 88.646) (width 0.25) (layer F.Cu) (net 3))
 (segment (start 46.863 95.504) (end 46.99 95.377) (width 0.25) (layer F.Cu) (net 4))
 (segment (start 46.99 95.377) (end 46.99 88.646) (width 0.25) (layer F.Cu) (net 4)))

